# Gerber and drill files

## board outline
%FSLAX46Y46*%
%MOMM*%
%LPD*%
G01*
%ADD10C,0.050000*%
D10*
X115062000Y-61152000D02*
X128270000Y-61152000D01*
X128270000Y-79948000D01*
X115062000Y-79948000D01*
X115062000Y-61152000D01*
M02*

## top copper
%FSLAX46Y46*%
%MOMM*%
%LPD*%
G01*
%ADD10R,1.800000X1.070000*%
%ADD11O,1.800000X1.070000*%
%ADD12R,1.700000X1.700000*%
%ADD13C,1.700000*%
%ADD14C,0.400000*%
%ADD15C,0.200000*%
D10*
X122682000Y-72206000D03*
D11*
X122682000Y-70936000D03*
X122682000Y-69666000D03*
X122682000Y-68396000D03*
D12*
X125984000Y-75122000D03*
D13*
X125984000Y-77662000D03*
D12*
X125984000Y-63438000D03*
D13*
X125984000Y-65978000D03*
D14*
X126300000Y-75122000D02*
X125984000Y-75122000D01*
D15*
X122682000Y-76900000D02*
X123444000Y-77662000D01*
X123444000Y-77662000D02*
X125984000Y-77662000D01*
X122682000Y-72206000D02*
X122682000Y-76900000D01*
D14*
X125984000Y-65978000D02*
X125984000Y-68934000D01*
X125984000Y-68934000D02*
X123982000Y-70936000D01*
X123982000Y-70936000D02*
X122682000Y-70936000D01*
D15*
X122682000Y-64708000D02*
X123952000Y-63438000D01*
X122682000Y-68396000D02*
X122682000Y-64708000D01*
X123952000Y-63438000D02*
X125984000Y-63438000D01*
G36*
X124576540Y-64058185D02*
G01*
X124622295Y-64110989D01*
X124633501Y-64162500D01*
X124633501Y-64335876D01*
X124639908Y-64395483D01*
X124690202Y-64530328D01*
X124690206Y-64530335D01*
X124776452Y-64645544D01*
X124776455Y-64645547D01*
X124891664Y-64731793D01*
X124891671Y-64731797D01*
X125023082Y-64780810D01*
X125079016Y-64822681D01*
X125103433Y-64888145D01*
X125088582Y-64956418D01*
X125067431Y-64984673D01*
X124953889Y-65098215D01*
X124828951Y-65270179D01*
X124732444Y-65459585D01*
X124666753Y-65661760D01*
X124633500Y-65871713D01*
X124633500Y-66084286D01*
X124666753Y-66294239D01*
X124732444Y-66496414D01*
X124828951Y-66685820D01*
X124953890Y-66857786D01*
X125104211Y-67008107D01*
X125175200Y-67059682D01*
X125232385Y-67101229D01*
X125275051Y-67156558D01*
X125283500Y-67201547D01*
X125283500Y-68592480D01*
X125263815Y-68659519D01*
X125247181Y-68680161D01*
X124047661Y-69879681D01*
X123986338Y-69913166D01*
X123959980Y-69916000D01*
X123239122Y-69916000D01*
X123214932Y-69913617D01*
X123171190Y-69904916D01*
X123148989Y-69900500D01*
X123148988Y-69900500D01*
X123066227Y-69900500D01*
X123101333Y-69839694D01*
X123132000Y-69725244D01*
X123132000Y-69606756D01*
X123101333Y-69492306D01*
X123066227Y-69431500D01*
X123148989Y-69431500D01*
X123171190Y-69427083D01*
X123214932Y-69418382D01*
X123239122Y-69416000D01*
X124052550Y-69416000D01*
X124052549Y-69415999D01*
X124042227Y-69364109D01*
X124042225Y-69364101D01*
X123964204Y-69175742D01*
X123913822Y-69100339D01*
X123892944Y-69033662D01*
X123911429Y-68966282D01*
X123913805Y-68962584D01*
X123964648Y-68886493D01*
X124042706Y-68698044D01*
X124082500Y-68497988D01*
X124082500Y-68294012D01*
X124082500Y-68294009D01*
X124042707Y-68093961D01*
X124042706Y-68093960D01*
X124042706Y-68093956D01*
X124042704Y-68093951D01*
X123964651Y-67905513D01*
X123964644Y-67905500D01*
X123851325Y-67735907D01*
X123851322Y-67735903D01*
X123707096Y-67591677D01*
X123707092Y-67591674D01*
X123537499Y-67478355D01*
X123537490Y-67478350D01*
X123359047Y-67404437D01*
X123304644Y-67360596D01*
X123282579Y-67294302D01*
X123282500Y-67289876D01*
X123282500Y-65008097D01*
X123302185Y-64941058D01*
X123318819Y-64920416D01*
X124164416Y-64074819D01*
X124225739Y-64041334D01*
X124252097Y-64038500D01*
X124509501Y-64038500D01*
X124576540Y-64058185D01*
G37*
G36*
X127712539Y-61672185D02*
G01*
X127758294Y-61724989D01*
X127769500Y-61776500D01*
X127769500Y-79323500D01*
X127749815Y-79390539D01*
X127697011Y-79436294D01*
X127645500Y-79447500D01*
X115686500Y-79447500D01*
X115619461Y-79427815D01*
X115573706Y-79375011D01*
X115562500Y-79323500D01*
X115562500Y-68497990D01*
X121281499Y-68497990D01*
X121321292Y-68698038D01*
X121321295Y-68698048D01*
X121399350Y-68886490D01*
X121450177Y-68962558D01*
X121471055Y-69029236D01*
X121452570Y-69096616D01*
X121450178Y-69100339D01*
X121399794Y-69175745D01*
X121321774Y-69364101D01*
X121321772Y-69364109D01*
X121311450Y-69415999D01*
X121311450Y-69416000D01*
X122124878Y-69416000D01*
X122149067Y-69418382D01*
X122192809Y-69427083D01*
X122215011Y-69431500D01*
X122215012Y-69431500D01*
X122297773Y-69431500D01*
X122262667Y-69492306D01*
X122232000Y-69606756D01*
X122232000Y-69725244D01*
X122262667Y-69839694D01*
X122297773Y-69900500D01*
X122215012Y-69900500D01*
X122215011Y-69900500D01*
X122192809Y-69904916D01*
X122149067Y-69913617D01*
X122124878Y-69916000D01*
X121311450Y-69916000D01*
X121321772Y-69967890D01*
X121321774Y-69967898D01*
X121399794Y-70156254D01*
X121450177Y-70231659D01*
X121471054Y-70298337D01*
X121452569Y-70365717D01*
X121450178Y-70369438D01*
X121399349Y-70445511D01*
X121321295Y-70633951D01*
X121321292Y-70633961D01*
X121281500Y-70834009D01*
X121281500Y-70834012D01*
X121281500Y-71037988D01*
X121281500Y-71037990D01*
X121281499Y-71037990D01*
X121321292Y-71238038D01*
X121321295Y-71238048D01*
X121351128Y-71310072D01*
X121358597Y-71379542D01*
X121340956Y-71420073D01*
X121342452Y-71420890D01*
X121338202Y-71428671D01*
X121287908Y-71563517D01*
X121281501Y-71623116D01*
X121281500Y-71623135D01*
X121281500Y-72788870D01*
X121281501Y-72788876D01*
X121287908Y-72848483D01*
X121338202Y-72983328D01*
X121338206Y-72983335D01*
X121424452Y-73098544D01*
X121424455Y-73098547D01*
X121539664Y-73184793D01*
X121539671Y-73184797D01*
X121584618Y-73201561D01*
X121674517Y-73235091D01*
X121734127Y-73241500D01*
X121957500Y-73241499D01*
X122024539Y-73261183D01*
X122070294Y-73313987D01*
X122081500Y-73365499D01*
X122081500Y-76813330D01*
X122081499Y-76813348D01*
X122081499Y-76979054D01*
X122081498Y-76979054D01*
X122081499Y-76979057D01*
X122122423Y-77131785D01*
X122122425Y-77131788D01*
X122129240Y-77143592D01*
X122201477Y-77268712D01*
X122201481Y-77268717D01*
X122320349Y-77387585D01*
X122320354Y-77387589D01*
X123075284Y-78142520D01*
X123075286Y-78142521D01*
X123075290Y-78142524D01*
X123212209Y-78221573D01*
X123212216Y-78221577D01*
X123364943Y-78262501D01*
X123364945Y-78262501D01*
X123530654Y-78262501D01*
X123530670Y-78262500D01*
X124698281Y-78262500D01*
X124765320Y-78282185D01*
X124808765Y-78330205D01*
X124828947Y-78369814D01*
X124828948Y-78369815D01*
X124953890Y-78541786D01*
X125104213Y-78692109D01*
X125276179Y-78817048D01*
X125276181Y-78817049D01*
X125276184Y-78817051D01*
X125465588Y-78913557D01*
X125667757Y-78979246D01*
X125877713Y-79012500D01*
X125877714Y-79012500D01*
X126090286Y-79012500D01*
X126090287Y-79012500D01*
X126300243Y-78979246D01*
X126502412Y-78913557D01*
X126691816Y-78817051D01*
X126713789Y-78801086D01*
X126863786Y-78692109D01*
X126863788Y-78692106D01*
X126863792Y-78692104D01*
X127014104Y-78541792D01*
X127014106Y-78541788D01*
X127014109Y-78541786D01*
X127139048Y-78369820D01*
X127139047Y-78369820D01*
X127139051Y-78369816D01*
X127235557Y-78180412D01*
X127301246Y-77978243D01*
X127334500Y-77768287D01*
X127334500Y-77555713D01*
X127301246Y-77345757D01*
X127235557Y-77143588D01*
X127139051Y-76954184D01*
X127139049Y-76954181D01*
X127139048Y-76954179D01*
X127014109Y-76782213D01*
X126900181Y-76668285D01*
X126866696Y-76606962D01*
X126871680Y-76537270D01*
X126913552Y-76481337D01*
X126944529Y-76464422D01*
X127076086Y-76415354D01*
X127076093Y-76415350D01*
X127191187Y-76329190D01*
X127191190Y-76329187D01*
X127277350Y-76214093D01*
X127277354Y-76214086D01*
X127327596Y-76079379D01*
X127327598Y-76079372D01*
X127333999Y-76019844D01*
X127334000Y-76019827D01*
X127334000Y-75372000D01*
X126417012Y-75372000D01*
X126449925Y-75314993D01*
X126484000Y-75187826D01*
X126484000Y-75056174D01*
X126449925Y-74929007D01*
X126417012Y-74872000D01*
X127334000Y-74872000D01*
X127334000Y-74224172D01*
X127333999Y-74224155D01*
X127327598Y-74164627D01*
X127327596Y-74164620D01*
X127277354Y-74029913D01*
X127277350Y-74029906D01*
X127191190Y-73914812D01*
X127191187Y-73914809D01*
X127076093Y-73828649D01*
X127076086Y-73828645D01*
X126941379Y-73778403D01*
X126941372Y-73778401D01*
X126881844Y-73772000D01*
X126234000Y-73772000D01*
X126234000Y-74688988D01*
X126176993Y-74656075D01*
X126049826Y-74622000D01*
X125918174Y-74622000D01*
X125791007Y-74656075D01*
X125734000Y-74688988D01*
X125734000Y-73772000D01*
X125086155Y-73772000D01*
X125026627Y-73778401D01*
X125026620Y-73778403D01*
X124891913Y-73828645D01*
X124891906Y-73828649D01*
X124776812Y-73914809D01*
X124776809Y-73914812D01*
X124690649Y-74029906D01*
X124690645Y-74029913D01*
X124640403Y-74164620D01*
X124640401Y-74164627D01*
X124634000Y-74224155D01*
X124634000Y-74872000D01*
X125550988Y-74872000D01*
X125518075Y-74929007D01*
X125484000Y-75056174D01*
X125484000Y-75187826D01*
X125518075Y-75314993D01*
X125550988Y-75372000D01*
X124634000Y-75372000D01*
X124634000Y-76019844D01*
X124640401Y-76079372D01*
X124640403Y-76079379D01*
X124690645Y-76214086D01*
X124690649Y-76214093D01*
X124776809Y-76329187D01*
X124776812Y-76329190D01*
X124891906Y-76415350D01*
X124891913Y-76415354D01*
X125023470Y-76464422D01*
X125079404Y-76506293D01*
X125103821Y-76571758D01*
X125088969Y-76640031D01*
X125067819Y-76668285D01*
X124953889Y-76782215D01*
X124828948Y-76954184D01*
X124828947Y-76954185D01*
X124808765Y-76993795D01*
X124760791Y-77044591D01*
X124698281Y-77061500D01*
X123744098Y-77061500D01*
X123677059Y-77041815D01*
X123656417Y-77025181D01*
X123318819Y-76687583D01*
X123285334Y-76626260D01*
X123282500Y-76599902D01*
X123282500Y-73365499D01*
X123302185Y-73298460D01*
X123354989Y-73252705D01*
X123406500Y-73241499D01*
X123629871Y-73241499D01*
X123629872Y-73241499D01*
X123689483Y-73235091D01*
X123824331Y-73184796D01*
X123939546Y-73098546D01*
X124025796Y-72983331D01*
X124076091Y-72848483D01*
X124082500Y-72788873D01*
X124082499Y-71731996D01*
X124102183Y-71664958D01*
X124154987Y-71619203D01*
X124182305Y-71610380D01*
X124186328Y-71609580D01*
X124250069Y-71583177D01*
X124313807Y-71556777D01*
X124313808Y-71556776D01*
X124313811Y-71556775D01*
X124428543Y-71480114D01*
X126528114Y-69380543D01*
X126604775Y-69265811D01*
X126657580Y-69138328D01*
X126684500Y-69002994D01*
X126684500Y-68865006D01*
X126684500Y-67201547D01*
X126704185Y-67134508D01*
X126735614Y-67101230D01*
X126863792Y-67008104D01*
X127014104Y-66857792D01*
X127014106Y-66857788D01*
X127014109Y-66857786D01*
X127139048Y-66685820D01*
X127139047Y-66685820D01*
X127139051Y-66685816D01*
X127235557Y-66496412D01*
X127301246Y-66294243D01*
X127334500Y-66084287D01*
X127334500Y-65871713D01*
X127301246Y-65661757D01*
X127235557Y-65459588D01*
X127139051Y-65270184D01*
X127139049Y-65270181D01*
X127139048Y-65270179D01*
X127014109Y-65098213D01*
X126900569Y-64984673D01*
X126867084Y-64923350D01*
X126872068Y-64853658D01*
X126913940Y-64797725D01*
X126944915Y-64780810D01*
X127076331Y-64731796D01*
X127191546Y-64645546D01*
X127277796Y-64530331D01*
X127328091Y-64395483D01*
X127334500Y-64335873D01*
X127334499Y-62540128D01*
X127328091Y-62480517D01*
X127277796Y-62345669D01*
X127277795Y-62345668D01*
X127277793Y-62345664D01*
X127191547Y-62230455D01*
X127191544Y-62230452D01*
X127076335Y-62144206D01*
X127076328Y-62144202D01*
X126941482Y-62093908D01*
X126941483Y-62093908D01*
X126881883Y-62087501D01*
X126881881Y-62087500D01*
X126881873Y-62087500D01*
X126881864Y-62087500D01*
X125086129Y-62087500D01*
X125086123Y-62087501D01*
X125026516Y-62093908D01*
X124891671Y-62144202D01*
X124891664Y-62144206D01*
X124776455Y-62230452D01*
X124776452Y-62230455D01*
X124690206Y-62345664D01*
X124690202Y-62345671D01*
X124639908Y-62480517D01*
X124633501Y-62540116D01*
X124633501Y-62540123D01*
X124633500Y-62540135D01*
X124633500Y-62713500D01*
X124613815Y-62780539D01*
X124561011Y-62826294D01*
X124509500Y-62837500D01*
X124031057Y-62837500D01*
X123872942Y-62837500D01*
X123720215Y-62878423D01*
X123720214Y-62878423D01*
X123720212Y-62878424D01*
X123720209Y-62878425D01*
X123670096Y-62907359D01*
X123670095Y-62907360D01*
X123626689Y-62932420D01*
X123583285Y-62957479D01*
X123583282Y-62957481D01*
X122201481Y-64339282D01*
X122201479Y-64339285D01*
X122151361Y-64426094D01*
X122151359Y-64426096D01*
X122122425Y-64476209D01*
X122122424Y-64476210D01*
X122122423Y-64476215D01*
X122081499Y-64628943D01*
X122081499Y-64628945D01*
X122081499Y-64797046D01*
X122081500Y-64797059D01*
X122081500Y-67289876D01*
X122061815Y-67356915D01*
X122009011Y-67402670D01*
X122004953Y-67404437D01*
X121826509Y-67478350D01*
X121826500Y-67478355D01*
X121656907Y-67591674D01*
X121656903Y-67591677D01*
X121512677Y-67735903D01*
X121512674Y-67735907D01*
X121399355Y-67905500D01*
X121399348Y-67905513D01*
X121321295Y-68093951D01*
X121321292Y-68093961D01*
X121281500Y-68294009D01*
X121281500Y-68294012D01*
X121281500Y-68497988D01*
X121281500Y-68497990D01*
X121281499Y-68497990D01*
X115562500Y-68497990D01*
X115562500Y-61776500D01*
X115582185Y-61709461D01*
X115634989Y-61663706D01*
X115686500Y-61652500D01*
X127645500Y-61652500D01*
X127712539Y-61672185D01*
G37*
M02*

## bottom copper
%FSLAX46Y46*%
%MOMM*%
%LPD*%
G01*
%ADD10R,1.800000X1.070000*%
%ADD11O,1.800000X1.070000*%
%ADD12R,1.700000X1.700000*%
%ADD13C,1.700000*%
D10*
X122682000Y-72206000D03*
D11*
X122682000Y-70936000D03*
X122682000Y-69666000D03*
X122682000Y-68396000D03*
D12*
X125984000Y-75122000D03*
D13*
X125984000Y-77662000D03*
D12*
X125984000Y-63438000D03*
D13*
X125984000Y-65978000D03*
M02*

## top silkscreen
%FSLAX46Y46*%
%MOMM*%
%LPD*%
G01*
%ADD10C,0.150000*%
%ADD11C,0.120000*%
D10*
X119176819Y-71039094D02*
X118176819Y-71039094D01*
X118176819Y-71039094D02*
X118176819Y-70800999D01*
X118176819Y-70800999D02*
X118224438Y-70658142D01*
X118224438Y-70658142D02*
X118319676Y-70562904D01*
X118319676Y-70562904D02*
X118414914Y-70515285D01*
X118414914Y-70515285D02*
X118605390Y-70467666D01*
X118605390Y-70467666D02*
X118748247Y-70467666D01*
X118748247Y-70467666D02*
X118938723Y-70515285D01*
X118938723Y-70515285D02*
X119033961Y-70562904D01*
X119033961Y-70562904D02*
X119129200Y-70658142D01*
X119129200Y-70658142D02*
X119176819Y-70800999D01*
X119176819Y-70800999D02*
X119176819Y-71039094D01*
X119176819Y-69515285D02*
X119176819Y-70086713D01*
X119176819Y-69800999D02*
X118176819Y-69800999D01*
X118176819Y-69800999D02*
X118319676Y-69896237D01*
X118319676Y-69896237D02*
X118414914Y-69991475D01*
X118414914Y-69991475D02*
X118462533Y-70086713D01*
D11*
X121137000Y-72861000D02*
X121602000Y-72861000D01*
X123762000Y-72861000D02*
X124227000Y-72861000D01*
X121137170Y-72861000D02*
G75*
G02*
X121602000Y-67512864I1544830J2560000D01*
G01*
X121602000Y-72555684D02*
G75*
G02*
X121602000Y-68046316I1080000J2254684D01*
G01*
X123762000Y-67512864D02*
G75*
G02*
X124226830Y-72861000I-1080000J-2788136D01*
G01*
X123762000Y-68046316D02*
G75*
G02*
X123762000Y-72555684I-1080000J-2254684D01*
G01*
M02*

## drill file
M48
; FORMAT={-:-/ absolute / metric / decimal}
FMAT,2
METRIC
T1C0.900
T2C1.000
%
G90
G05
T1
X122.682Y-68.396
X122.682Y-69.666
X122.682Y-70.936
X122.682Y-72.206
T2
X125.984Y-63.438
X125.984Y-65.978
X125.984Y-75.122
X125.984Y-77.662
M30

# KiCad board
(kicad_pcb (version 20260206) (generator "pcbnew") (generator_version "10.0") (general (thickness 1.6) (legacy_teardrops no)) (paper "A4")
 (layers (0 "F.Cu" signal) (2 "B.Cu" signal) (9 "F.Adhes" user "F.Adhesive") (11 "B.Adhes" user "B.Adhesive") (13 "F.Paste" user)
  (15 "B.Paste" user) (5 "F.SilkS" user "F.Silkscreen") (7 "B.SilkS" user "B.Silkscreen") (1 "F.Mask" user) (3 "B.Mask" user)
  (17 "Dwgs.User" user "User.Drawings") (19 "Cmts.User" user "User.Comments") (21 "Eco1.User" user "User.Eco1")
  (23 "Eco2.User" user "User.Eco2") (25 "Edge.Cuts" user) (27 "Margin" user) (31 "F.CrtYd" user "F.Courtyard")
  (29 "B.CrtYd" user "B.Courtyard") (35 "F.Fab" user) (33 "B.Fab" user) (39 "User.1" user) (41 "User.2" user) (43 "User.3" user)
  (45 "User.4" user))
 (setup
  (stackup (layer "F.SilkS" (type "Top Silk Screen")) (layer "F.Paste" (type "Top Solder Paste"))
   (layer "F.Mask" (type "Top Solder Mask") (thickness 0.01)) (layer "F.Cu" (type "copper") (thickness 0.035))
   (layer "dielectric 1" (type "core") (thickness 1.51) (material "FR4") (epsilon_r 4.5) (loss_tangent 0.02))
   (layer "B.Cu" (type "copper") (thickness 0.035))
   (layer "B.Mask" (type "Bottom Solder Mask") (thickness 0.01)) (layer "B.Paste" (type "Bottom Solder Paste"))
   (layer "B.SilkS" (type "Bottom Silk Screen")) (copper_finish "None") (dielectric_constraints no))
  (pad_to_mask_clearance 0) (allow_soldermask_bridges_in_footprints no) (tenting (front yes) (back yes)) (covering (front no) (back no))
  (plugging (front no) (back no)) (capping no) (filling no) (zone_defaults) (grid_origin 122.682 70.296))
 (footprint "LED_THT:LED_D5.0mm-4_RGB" (layer "F.Cu") (at 122.682 72.206 90)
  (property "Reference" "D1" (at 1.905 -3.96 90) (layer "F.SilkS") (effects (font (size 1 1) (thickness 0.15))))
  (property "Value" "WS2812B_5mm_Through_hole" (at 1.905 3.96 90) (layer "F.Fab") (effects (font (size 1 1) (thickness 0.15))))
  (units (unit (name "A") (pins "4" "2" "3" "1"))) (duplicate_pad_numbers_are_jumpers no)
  (fp_line (start -0.655 -1.545) (end -0.655 -1.08) (stroke (width 0.12) (type solid)) (layer "F.SilkS"))
  (fp_line (start -0.655 1.08) (end -0.655 1.545) (stroke (width 0.12) (type solid)) (layer "F.SilkS"))
  (fp_arc (start -0.655 -1.54483) (mid 2.163898 -2.97877) (end 4.693136 -1.08) (stroke (width 0.12) (type solid)) (layer "F.SilkS"))
  (fp_arc (start -0.349684 -1.08) (mid 1.905 -2.5) (end 4.159684 -1.08) (stroke (width 0.12) (type solid)) (layer "F.SilkS"))
  (fp_arc (start 4.693136 1.08) (mid 2.163898 2.97877) (end -0.655 1.54483) (stroke (width 0.12) (type solid)) (layer "F.SilkS"))
  (fp_arc (start 4.159684 1.08) (mid 1.905 2.5) (end -0.349684 1.08) (stroke (width 0.12) (type solid)) (layer "F.SilkS"))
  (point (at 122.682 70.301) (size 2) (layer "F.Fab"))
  (pad "1" thru_hole rect (at 0 0 90) (size 1.07 1.8) (drill 0.9) (layers "*.Cu" "*.Mask") (remove_unused_layers no) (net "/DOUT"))
  (pad "2" thru_hole oval (at 1.27 0 90) (size 1.07 1.8) (drill 0.9) (layers "*.Cu" "*.Mask") (remove_unused_layers no) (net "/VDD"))
  (pad "3" thru_hole oval (at 2.54 0 90) (size 1.07 1.8) (drill 0.9) (layers "*.Cu" "*.Mask") (remove_unused_layers no) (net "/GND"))
  (pad "4" thru_hole oval (at 3.81 0 90) (size 1.07 1.8) (drill 0.9) (layers "*.Cu" "*.Mask") (remove_unused_layers no) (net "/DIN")))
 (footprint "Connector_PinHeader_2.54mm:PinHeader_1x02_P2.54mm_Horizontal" (layer "B.Cu") (at 125.984 75.122 180)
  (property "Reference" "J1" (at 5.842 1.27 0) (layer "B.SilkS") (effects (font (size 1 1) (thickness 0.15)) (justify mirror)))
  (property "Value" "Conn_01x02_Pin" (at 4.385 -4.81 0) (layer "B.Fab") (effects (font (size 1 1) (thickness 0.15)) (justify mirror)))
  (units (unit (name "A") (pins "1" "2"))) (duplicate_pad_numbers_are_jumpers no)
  (pad "1" thru_hole rect (at 0 0 180) (size 1.7 1.7) (drill 1) (layers "*.Cu" "*.Mask") (remove_unused_layers no) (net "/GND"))
  (pad "2" thru_hole circle (at 0 -2.54 180) (size 1.7 1.7) (drill 1) (layers "*.Cu" "*.Mask") (remove_unused_layers no) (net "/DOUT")))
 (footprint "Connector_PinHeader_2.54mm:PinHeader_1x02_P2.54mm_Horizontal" (layer "B.Cu") (at 125.984 63.438 180)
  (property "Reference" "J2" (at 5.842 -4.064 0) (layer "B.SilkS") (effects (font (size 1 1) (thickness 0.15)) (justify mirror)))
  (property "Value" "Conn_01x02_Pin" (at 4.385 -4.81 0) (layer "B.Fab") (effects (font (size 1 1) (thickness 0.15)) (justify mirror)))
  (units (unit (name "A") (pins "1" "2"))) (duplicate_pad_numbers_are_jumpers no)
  (pad "1" thru_hole rect (at 0 0 180) (size 1.7 1.7) (drill 1) (layers "*.Cu" "*.Mask") (remove_unused_layers no) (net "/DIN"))
  (pad "2" thru_hole circle (at 0 -2.54 180) (size 1.7 1.7) (drill 1) (layers "*.Cu" "*.Mask") (remove_unused_layers no) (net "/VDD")))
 (gr_rect (start 115.062 61.152) (end 128.27 79.948) (stroke (width 0.05) (type default)) (fill no) (layer "Edge.Cuts"))
 (segment (start 126.3 75.122) (end 125.984 75.122) (width 0.4) (layer "F.Cu") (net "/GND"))
 (segment (start 122.682 76.9) (end 123.444 77.662) (width 0.2) (layer "F.Cu") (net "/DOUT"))
 (segment (start 123.444 77.662) (end 125.984 77.662) (width 0.2) (layer "F.Cu") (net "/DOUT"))
 (segment (start 122.682 72.206) (end 122.682 76.9) (width 0.2) (layer "F.Cu") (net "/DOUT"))
 (segment (start 125.984 65.978) (end 125.984 68.934) (width 0.4) (layer "F.Cu") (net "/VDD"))
 (segment (start 125.984 68.934) (end 123.982 70.936) (width 0.4) (layer "F.Cu") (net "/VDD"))
 (segment (start 123.982 70.936) (end 122.682 70.936) (width 0.4) (layer "F.Cu") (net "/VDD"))
 (segment (start 122.682 64.708) (end 123.952 63.438) (width 0.2) (layer "F.Cu") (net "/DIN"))
 (segment (start 122.682 68.396) (end 122.682 64.708) (width 0.2) (layer "F.Cu") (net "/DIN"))
 (segment (start 123.952 63.438) (end 125.984 63.438) (width 0.2) (layer "F.Cu") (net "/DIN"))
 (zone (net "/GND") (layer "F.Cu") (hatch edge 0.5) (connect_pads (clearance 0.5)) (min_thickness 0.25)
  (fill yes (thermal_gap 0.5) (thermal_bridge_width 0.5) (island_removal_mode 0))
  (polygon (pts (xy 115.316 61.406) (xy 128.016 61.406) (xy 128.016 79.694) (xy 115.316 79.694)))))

